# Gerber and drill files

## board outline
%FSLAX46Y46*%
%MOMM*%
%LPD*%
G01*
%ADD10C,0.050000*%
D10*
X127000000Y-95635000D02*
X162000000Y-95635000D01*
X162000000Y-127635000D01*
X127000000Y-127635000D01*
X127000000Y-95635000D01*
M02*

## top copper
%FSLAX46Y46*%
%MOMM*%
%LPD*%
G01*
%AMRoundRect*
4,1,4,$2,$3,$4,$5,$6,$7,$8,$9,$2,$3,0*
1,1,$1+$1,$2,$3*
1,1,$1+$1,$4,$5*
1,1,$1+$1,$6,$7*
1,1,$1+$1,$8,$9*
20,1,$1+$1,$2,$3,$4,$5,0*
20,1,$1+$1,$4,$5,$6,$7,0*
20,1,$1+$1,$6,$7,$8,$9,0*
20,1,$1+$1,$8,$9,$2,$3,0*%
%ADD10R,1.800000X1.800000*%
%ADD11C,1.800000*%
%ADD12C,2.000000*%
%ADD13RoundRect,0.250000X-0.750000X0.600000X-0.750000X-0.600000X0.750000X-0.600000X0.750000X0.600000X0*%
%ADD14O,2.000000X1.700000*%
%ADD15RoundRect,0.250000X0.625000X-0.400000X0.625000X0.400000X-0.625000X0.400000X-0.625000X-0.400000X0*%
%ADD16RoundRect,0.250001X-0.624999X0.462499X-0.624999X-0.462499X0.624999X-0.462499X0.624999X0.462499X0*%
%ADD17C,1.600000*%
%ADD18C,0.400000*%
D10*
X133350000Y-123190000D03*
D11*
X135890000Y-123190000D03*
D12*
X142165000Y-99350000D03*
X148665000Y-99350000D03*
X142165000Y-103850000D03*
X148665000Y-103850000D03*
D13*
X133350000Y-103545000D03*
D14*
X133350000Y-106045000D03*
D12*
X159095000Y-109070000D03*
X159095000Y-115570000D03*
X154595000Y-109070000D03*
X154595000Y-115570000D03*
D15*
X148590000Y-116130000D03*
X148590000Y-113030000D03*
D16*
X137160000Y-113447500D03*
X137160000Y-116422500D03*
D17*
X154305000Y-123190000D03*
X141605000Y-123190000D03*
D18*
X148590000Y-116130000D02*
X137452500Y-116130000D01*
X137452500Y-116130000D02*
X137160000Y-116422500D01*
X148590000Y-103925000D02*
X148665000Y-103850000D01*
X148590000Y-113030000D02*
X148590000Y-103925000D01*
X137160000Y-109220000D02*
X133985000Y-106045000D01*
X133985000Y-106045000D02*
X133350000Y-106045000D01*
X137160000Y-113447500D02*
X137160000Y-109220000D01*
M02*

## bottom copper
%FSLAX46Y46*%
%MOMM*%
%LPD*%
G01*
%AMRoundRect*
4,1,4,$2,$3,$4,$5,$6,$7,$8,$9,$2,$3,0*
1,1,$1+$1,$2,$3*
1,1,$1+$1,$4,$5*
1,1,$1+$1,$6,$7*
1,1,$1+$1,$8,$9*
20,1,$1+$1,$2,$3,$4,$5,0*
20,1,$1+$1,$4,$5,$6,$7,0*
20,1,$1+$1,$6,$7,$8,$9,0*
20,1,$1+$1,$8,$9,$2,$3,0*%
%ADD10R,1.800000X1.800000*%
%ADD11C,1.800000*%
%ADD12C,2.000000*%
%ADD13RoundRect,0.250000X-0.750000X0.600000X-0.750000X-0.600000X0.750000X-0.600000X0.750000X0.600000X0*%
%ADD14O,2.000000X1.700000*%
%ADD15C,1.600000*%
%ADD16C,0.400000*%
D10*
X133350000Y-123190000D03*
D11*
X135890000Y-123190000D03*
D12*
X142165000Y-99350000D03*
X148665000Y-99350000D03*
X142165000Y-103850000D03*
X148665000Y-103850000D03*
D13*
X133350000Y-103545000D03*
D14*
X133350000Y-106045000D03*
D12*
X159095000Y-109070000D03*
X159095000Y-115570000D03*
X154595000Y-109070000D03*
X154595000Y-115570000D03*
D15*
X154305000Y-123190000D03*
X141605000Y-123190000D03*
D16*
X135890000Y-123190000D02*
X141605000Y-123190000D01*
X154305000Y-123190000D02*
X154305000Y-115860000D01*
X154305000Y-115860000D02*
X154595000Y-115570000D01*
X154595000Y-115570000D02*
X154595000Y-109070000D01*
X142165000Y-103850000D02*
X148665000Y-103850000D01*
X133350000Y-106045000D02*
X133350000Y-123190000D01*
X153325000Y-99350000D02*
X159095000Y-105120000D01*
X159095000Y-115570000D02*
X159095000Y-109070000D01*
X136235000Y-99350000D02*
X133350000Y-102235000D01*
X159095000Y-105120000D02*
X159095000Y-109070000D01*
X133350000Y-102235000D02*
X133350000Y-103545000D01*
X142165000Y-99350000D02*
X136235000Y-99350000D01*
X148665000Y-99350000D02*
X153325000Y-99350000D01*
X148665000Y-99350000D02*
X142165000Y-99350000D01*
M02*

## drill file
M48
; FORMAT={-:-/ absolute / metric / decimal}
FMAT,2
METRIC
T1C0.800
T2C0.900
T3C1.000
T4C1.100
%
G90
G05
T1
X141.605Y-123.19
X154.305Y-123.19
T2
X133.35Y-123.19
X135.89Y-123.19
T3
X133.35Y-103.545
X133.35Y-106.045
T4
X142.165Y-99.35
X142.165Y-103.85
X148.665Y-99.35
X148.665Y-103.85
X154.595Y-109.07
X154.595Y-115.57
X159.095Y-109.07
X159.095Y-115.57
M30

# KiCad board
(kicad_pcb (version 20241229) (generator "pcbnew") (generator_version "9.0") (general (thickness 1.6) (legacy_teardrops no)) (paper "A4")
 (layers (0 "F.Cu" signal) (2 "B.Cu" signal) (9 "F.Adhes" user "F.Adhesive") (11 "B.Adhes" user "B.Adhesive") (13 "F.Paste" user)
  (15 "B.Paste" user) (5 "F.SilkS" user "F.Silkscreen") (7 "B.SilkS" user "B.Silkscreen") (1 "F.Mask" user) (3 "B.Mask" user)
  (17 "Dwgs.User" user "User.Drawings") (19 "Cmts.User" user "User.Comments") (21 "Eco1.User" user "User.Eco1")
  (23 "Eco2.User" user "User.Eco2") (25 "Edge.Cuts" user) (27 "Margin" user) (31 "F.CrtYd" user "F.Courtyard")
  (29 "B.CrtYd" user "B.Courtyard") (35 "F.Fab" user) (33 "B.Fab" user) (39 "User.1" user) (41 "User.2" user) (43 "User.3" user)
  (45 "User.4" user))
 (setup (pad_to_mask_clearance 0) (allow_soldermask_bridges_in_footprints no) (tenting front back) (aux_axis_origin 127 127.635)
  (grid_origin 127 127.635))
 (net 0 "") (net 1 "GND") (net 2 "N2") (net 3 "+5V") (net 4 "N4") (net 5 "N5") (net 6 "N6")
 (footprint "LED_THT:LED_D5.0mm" (layer "F.Cu") (at 133.35 123.19)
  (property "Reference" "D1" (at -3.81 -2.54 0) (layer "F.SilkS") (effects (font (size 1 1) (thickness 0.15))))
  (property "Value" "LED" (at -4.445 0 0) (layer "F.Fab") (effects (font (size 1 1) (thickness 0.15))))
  (pad "1" thru_hole rect (at 0 0) (size 1.8 1.8) (drill 0.9) (layers "*.Cu" "*.Mask") (remove_unused_layers no) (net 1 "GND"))
  (pad "2" thru_hole circle (at 2.54 0) (size 1.8 1.8) (drill 0.9) (layers "*.Cu" "*.Mask") (remove_unused_layers no) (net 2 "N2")))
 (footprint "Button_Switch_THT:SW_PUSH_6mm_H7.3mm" (layer "F.Cu") (at 142.165 99.35)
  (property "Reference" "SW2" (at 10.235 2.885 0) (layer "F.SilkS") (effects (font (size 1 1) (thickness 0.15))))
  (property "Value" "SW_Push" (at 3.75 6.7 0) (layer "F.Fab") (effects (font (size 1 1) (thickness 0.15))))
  (pad "1" thru_hole circle (at 0 0 90) (size 2 2) (drill 1.1) (layers "*.Cu" "*.Mask") (remove_unused_layers no) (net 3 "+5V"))
  (pad "1" thru_hole circle (at 6.5 0 90) (size 2 2) (drill 1.1) (layers "*.Cu" "*.Mask") (remove_unused_layers no) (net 3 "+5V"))
  (pad "2" thru_hole circle (at 0 4.5 90) (size 2 2) (drill 1.1) (layers "*.Cu" "*.Mask") (remove_unused_layers no) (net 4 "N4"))
  (pad "2" thru_hole circle (at 6.5 4.5 90) (size 2 2) (drill 1.1) (layers "*.Cu" "*.Mask") (remove_unused_layers no) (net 4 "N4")))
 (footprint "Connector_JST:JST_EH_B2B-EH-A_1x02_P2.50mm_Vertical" (layer "F.Cu") (at 133.35 103.545 -90)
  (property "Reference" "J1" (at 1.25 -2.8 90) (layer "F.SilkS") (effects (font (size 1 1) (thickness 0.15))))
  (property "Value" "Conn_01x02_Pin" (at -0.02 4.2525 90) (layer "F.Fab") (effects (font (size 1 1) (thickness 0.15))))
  (pad "1" thru_hole roundrect (at 0 0 270) (size 1.7 2) (drill 1) (layers "*.Cu" "*.Mask") (remove_unused_layers no)
   (roundrect_rratio 0.147059) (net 3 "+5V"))
  (pad "2" thru_hole oval (at 2.5 0 270) (size 1.7 2) (drill 1) (layers "*.Cu" "*.Mask") (remove_unused_layers no) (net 1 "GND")))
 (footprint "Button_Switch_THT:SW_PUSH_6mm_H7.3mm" (layer "F.Cu") (at 159.095 109.07 -90)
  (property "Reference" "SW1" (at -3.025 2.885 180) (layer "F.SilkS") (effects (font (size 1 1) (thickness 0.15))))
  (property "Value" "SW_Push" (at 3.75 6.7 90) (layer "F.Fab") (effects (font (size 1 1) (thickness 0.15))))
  (pad "1" thru_hole circle (at 0 0) (size 2 2) (drill 1.1) (layers "*.Cu" "*.Mask") (remove_unused_layers no) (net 3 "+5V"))
  (pad "1" thru_hole circle (at 6.5 0) (size 2 2) (drill 1.1) (layers "*.Cu" "*.Mask") (remove_unused_layers no) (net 3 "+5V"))
  (pad "2" thru_hole circle (at 0 4.5) (size 2 2) (drill 1.1) (layers "*.Cu" "*.Mask") (remove_unused_layers no) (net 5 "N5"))
  (pad "2" thru_hole circle (at 6.5 4.5) (size 2 2) (drill 1.1) (layers "*.Cu" "*.Mask") (remove_unused_layers no) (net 5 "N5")))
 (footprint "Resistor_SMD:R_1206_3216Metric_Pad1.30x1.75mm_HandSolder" (layer "F.Cu") (at 148.59 114.58 90)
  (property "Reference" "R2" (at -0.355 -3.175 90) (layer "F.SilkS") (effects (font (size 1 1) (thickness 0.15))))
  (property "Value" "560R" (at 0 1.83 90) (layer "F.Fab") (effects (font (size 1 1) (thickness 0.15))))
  (pad "1" smd roundrect (at -1.55 0 90) (size 1.3 1.75) (layers "F.Cu" "F.Mask" "F.Paste") (roundrect_rratio 0.192308) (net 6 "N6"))
  (pad "2" smd roundrect (at 1.55 0 90) (size 1.3 1.75) (layers "F.Cu" "F.Mask" "F.Paste") (roundrect_rratio 0.192308) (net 4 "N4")))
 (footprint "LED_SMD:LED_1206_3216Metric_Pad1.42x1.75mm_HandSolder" (layer "F.Cu") (at 137.16 114.935 -90)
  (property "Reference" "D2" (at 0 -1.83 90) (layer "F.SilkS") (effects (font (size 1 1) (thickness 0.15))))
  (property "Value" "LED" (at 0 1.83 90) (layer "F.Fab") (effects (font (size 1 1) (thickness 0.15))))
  (pad "1" smd roundrect (at -1.4875 0 270) (size 1.425 1.75) (layers "F.Cu" "F.Mask" "F.Paste") (roundrect_rratio 0.175439) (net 1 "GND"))
  (pad "2" smd roundrect (at 1.4875 0 270) (size 1.425 1.75) (layers "F.Cu" "F.Mask" "F.Paste") (roundrect_rratio 0.175439) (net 6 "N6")))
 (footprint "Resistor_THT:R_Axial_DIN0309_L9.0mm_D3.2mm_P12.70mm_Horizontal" (layer "F.Cu") (at 154.305 123.19 180)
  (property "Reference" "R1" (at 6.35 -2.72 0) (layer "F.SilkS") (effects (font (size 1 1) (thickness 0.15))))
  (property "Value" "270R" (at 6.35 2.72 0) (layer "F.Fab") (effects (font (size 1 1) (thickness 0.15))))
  (pad "1" thru_hole circle (at 0 0 180) (size 1.6 1.6) (drill 0.8) (layers "*.Cu" "*.Mask") (remove_unused_layers no) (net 5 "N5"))
  (pad "2" thru_hole circle (at 12.7 0 180) (size 1.6 1.6) (drill 0.8) (layers "*.Cu" "*.Mask") (remove_unused_layers no) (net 2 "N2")))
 (gr_rect (start 127 95.635) (end 162 127.635) (stroke (width 0.05) (type solid)) (fill no) (layer "Edge.Cuts"))
 (segment (start 135.89 123.19) (end 141.605 123.19) (width 0.4) (layer "B.Cu") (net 2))
 (segment (start 148.59 116.13) (end 137.4525 116.13) (width 0.4) (layer "F.Cu") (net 6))
 (segment (start 137.4525 116.13) (end 137.16 116.4225) (width 0.4) (layer "F.Cu") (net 6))
 (segment (start 154.305 123.19) (end 154.305 115.86) (width 0.4) (layer "B.Cu") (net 5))
 (segment (start 154.305 115.86) (end 154.595 115.57) (width 0.4) (layer "B.Cu") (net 5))
 (segment (start 154.595 115.57) (end 154.595 109.07) (width 0.4) (layer "B.Cu") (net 5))
 (segment (start 148.59 103.925) (end 148.665 103.85) (width 0.4) (layer "F.Cu") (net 4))
 (segment (start 148.59 113.03) (end 148.59 103.925) (width 0.4) (layer "F.Cu") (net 4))
 (segment (start 142.165 103.85) (end 148.665 103.85) (width 0.4) (layer "B.Cu") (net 4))
 (segment (start 137.16 109.22) (end 133.985 106.045) (width 0.4) (layer "F.Cu") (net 1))
 (segment (start 133.985 106.045) (end 133.35 106.045) (width 0.4) (layer "F.Cu") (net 1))
 (segment (start 137.16 113.4475) (end 137.16 109.22) (width 0.4) (layer "F.Cu") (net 1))
 (segment (start 133.35 106.045) (end 133.35 123.19) (width 0.4) (layer "B.Cu") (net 1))
 (segment (start 153.325 99.35) (end 159.095 105.12) (width 0.4) (layer "B.Cu") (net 3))
 (segment (start 159.095 115.57) (end 159.095 109.07) (width 0.4) (layer "B.Cu") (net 3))
 (segment (start 136.235 99.35) (end 133.35 102.235) (width 0.4) (layer "B.Cu") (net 3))
 (segment (start 159.095 105.12) (end 159.095 109.07) (width 0.4) (layer "B.Cu") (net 3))
 (segment (start 133.35 102.235) (end 133.35 103.545) (width 0.4) (layer "B.Cu") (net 3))
 (segment (start 142.165 99.35) (end 136.235 99.35) (width 0.4) (layer "B.Cu") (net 3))
 (segment (start 148.665 99.35) (end 153.325 99.35) (width 0.4) (layer "B.Cu") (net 3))
 (segment (start 148.665 99.35) (end 142.165 99.35) (width 0.4) (layer "B.Cu") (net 3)))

